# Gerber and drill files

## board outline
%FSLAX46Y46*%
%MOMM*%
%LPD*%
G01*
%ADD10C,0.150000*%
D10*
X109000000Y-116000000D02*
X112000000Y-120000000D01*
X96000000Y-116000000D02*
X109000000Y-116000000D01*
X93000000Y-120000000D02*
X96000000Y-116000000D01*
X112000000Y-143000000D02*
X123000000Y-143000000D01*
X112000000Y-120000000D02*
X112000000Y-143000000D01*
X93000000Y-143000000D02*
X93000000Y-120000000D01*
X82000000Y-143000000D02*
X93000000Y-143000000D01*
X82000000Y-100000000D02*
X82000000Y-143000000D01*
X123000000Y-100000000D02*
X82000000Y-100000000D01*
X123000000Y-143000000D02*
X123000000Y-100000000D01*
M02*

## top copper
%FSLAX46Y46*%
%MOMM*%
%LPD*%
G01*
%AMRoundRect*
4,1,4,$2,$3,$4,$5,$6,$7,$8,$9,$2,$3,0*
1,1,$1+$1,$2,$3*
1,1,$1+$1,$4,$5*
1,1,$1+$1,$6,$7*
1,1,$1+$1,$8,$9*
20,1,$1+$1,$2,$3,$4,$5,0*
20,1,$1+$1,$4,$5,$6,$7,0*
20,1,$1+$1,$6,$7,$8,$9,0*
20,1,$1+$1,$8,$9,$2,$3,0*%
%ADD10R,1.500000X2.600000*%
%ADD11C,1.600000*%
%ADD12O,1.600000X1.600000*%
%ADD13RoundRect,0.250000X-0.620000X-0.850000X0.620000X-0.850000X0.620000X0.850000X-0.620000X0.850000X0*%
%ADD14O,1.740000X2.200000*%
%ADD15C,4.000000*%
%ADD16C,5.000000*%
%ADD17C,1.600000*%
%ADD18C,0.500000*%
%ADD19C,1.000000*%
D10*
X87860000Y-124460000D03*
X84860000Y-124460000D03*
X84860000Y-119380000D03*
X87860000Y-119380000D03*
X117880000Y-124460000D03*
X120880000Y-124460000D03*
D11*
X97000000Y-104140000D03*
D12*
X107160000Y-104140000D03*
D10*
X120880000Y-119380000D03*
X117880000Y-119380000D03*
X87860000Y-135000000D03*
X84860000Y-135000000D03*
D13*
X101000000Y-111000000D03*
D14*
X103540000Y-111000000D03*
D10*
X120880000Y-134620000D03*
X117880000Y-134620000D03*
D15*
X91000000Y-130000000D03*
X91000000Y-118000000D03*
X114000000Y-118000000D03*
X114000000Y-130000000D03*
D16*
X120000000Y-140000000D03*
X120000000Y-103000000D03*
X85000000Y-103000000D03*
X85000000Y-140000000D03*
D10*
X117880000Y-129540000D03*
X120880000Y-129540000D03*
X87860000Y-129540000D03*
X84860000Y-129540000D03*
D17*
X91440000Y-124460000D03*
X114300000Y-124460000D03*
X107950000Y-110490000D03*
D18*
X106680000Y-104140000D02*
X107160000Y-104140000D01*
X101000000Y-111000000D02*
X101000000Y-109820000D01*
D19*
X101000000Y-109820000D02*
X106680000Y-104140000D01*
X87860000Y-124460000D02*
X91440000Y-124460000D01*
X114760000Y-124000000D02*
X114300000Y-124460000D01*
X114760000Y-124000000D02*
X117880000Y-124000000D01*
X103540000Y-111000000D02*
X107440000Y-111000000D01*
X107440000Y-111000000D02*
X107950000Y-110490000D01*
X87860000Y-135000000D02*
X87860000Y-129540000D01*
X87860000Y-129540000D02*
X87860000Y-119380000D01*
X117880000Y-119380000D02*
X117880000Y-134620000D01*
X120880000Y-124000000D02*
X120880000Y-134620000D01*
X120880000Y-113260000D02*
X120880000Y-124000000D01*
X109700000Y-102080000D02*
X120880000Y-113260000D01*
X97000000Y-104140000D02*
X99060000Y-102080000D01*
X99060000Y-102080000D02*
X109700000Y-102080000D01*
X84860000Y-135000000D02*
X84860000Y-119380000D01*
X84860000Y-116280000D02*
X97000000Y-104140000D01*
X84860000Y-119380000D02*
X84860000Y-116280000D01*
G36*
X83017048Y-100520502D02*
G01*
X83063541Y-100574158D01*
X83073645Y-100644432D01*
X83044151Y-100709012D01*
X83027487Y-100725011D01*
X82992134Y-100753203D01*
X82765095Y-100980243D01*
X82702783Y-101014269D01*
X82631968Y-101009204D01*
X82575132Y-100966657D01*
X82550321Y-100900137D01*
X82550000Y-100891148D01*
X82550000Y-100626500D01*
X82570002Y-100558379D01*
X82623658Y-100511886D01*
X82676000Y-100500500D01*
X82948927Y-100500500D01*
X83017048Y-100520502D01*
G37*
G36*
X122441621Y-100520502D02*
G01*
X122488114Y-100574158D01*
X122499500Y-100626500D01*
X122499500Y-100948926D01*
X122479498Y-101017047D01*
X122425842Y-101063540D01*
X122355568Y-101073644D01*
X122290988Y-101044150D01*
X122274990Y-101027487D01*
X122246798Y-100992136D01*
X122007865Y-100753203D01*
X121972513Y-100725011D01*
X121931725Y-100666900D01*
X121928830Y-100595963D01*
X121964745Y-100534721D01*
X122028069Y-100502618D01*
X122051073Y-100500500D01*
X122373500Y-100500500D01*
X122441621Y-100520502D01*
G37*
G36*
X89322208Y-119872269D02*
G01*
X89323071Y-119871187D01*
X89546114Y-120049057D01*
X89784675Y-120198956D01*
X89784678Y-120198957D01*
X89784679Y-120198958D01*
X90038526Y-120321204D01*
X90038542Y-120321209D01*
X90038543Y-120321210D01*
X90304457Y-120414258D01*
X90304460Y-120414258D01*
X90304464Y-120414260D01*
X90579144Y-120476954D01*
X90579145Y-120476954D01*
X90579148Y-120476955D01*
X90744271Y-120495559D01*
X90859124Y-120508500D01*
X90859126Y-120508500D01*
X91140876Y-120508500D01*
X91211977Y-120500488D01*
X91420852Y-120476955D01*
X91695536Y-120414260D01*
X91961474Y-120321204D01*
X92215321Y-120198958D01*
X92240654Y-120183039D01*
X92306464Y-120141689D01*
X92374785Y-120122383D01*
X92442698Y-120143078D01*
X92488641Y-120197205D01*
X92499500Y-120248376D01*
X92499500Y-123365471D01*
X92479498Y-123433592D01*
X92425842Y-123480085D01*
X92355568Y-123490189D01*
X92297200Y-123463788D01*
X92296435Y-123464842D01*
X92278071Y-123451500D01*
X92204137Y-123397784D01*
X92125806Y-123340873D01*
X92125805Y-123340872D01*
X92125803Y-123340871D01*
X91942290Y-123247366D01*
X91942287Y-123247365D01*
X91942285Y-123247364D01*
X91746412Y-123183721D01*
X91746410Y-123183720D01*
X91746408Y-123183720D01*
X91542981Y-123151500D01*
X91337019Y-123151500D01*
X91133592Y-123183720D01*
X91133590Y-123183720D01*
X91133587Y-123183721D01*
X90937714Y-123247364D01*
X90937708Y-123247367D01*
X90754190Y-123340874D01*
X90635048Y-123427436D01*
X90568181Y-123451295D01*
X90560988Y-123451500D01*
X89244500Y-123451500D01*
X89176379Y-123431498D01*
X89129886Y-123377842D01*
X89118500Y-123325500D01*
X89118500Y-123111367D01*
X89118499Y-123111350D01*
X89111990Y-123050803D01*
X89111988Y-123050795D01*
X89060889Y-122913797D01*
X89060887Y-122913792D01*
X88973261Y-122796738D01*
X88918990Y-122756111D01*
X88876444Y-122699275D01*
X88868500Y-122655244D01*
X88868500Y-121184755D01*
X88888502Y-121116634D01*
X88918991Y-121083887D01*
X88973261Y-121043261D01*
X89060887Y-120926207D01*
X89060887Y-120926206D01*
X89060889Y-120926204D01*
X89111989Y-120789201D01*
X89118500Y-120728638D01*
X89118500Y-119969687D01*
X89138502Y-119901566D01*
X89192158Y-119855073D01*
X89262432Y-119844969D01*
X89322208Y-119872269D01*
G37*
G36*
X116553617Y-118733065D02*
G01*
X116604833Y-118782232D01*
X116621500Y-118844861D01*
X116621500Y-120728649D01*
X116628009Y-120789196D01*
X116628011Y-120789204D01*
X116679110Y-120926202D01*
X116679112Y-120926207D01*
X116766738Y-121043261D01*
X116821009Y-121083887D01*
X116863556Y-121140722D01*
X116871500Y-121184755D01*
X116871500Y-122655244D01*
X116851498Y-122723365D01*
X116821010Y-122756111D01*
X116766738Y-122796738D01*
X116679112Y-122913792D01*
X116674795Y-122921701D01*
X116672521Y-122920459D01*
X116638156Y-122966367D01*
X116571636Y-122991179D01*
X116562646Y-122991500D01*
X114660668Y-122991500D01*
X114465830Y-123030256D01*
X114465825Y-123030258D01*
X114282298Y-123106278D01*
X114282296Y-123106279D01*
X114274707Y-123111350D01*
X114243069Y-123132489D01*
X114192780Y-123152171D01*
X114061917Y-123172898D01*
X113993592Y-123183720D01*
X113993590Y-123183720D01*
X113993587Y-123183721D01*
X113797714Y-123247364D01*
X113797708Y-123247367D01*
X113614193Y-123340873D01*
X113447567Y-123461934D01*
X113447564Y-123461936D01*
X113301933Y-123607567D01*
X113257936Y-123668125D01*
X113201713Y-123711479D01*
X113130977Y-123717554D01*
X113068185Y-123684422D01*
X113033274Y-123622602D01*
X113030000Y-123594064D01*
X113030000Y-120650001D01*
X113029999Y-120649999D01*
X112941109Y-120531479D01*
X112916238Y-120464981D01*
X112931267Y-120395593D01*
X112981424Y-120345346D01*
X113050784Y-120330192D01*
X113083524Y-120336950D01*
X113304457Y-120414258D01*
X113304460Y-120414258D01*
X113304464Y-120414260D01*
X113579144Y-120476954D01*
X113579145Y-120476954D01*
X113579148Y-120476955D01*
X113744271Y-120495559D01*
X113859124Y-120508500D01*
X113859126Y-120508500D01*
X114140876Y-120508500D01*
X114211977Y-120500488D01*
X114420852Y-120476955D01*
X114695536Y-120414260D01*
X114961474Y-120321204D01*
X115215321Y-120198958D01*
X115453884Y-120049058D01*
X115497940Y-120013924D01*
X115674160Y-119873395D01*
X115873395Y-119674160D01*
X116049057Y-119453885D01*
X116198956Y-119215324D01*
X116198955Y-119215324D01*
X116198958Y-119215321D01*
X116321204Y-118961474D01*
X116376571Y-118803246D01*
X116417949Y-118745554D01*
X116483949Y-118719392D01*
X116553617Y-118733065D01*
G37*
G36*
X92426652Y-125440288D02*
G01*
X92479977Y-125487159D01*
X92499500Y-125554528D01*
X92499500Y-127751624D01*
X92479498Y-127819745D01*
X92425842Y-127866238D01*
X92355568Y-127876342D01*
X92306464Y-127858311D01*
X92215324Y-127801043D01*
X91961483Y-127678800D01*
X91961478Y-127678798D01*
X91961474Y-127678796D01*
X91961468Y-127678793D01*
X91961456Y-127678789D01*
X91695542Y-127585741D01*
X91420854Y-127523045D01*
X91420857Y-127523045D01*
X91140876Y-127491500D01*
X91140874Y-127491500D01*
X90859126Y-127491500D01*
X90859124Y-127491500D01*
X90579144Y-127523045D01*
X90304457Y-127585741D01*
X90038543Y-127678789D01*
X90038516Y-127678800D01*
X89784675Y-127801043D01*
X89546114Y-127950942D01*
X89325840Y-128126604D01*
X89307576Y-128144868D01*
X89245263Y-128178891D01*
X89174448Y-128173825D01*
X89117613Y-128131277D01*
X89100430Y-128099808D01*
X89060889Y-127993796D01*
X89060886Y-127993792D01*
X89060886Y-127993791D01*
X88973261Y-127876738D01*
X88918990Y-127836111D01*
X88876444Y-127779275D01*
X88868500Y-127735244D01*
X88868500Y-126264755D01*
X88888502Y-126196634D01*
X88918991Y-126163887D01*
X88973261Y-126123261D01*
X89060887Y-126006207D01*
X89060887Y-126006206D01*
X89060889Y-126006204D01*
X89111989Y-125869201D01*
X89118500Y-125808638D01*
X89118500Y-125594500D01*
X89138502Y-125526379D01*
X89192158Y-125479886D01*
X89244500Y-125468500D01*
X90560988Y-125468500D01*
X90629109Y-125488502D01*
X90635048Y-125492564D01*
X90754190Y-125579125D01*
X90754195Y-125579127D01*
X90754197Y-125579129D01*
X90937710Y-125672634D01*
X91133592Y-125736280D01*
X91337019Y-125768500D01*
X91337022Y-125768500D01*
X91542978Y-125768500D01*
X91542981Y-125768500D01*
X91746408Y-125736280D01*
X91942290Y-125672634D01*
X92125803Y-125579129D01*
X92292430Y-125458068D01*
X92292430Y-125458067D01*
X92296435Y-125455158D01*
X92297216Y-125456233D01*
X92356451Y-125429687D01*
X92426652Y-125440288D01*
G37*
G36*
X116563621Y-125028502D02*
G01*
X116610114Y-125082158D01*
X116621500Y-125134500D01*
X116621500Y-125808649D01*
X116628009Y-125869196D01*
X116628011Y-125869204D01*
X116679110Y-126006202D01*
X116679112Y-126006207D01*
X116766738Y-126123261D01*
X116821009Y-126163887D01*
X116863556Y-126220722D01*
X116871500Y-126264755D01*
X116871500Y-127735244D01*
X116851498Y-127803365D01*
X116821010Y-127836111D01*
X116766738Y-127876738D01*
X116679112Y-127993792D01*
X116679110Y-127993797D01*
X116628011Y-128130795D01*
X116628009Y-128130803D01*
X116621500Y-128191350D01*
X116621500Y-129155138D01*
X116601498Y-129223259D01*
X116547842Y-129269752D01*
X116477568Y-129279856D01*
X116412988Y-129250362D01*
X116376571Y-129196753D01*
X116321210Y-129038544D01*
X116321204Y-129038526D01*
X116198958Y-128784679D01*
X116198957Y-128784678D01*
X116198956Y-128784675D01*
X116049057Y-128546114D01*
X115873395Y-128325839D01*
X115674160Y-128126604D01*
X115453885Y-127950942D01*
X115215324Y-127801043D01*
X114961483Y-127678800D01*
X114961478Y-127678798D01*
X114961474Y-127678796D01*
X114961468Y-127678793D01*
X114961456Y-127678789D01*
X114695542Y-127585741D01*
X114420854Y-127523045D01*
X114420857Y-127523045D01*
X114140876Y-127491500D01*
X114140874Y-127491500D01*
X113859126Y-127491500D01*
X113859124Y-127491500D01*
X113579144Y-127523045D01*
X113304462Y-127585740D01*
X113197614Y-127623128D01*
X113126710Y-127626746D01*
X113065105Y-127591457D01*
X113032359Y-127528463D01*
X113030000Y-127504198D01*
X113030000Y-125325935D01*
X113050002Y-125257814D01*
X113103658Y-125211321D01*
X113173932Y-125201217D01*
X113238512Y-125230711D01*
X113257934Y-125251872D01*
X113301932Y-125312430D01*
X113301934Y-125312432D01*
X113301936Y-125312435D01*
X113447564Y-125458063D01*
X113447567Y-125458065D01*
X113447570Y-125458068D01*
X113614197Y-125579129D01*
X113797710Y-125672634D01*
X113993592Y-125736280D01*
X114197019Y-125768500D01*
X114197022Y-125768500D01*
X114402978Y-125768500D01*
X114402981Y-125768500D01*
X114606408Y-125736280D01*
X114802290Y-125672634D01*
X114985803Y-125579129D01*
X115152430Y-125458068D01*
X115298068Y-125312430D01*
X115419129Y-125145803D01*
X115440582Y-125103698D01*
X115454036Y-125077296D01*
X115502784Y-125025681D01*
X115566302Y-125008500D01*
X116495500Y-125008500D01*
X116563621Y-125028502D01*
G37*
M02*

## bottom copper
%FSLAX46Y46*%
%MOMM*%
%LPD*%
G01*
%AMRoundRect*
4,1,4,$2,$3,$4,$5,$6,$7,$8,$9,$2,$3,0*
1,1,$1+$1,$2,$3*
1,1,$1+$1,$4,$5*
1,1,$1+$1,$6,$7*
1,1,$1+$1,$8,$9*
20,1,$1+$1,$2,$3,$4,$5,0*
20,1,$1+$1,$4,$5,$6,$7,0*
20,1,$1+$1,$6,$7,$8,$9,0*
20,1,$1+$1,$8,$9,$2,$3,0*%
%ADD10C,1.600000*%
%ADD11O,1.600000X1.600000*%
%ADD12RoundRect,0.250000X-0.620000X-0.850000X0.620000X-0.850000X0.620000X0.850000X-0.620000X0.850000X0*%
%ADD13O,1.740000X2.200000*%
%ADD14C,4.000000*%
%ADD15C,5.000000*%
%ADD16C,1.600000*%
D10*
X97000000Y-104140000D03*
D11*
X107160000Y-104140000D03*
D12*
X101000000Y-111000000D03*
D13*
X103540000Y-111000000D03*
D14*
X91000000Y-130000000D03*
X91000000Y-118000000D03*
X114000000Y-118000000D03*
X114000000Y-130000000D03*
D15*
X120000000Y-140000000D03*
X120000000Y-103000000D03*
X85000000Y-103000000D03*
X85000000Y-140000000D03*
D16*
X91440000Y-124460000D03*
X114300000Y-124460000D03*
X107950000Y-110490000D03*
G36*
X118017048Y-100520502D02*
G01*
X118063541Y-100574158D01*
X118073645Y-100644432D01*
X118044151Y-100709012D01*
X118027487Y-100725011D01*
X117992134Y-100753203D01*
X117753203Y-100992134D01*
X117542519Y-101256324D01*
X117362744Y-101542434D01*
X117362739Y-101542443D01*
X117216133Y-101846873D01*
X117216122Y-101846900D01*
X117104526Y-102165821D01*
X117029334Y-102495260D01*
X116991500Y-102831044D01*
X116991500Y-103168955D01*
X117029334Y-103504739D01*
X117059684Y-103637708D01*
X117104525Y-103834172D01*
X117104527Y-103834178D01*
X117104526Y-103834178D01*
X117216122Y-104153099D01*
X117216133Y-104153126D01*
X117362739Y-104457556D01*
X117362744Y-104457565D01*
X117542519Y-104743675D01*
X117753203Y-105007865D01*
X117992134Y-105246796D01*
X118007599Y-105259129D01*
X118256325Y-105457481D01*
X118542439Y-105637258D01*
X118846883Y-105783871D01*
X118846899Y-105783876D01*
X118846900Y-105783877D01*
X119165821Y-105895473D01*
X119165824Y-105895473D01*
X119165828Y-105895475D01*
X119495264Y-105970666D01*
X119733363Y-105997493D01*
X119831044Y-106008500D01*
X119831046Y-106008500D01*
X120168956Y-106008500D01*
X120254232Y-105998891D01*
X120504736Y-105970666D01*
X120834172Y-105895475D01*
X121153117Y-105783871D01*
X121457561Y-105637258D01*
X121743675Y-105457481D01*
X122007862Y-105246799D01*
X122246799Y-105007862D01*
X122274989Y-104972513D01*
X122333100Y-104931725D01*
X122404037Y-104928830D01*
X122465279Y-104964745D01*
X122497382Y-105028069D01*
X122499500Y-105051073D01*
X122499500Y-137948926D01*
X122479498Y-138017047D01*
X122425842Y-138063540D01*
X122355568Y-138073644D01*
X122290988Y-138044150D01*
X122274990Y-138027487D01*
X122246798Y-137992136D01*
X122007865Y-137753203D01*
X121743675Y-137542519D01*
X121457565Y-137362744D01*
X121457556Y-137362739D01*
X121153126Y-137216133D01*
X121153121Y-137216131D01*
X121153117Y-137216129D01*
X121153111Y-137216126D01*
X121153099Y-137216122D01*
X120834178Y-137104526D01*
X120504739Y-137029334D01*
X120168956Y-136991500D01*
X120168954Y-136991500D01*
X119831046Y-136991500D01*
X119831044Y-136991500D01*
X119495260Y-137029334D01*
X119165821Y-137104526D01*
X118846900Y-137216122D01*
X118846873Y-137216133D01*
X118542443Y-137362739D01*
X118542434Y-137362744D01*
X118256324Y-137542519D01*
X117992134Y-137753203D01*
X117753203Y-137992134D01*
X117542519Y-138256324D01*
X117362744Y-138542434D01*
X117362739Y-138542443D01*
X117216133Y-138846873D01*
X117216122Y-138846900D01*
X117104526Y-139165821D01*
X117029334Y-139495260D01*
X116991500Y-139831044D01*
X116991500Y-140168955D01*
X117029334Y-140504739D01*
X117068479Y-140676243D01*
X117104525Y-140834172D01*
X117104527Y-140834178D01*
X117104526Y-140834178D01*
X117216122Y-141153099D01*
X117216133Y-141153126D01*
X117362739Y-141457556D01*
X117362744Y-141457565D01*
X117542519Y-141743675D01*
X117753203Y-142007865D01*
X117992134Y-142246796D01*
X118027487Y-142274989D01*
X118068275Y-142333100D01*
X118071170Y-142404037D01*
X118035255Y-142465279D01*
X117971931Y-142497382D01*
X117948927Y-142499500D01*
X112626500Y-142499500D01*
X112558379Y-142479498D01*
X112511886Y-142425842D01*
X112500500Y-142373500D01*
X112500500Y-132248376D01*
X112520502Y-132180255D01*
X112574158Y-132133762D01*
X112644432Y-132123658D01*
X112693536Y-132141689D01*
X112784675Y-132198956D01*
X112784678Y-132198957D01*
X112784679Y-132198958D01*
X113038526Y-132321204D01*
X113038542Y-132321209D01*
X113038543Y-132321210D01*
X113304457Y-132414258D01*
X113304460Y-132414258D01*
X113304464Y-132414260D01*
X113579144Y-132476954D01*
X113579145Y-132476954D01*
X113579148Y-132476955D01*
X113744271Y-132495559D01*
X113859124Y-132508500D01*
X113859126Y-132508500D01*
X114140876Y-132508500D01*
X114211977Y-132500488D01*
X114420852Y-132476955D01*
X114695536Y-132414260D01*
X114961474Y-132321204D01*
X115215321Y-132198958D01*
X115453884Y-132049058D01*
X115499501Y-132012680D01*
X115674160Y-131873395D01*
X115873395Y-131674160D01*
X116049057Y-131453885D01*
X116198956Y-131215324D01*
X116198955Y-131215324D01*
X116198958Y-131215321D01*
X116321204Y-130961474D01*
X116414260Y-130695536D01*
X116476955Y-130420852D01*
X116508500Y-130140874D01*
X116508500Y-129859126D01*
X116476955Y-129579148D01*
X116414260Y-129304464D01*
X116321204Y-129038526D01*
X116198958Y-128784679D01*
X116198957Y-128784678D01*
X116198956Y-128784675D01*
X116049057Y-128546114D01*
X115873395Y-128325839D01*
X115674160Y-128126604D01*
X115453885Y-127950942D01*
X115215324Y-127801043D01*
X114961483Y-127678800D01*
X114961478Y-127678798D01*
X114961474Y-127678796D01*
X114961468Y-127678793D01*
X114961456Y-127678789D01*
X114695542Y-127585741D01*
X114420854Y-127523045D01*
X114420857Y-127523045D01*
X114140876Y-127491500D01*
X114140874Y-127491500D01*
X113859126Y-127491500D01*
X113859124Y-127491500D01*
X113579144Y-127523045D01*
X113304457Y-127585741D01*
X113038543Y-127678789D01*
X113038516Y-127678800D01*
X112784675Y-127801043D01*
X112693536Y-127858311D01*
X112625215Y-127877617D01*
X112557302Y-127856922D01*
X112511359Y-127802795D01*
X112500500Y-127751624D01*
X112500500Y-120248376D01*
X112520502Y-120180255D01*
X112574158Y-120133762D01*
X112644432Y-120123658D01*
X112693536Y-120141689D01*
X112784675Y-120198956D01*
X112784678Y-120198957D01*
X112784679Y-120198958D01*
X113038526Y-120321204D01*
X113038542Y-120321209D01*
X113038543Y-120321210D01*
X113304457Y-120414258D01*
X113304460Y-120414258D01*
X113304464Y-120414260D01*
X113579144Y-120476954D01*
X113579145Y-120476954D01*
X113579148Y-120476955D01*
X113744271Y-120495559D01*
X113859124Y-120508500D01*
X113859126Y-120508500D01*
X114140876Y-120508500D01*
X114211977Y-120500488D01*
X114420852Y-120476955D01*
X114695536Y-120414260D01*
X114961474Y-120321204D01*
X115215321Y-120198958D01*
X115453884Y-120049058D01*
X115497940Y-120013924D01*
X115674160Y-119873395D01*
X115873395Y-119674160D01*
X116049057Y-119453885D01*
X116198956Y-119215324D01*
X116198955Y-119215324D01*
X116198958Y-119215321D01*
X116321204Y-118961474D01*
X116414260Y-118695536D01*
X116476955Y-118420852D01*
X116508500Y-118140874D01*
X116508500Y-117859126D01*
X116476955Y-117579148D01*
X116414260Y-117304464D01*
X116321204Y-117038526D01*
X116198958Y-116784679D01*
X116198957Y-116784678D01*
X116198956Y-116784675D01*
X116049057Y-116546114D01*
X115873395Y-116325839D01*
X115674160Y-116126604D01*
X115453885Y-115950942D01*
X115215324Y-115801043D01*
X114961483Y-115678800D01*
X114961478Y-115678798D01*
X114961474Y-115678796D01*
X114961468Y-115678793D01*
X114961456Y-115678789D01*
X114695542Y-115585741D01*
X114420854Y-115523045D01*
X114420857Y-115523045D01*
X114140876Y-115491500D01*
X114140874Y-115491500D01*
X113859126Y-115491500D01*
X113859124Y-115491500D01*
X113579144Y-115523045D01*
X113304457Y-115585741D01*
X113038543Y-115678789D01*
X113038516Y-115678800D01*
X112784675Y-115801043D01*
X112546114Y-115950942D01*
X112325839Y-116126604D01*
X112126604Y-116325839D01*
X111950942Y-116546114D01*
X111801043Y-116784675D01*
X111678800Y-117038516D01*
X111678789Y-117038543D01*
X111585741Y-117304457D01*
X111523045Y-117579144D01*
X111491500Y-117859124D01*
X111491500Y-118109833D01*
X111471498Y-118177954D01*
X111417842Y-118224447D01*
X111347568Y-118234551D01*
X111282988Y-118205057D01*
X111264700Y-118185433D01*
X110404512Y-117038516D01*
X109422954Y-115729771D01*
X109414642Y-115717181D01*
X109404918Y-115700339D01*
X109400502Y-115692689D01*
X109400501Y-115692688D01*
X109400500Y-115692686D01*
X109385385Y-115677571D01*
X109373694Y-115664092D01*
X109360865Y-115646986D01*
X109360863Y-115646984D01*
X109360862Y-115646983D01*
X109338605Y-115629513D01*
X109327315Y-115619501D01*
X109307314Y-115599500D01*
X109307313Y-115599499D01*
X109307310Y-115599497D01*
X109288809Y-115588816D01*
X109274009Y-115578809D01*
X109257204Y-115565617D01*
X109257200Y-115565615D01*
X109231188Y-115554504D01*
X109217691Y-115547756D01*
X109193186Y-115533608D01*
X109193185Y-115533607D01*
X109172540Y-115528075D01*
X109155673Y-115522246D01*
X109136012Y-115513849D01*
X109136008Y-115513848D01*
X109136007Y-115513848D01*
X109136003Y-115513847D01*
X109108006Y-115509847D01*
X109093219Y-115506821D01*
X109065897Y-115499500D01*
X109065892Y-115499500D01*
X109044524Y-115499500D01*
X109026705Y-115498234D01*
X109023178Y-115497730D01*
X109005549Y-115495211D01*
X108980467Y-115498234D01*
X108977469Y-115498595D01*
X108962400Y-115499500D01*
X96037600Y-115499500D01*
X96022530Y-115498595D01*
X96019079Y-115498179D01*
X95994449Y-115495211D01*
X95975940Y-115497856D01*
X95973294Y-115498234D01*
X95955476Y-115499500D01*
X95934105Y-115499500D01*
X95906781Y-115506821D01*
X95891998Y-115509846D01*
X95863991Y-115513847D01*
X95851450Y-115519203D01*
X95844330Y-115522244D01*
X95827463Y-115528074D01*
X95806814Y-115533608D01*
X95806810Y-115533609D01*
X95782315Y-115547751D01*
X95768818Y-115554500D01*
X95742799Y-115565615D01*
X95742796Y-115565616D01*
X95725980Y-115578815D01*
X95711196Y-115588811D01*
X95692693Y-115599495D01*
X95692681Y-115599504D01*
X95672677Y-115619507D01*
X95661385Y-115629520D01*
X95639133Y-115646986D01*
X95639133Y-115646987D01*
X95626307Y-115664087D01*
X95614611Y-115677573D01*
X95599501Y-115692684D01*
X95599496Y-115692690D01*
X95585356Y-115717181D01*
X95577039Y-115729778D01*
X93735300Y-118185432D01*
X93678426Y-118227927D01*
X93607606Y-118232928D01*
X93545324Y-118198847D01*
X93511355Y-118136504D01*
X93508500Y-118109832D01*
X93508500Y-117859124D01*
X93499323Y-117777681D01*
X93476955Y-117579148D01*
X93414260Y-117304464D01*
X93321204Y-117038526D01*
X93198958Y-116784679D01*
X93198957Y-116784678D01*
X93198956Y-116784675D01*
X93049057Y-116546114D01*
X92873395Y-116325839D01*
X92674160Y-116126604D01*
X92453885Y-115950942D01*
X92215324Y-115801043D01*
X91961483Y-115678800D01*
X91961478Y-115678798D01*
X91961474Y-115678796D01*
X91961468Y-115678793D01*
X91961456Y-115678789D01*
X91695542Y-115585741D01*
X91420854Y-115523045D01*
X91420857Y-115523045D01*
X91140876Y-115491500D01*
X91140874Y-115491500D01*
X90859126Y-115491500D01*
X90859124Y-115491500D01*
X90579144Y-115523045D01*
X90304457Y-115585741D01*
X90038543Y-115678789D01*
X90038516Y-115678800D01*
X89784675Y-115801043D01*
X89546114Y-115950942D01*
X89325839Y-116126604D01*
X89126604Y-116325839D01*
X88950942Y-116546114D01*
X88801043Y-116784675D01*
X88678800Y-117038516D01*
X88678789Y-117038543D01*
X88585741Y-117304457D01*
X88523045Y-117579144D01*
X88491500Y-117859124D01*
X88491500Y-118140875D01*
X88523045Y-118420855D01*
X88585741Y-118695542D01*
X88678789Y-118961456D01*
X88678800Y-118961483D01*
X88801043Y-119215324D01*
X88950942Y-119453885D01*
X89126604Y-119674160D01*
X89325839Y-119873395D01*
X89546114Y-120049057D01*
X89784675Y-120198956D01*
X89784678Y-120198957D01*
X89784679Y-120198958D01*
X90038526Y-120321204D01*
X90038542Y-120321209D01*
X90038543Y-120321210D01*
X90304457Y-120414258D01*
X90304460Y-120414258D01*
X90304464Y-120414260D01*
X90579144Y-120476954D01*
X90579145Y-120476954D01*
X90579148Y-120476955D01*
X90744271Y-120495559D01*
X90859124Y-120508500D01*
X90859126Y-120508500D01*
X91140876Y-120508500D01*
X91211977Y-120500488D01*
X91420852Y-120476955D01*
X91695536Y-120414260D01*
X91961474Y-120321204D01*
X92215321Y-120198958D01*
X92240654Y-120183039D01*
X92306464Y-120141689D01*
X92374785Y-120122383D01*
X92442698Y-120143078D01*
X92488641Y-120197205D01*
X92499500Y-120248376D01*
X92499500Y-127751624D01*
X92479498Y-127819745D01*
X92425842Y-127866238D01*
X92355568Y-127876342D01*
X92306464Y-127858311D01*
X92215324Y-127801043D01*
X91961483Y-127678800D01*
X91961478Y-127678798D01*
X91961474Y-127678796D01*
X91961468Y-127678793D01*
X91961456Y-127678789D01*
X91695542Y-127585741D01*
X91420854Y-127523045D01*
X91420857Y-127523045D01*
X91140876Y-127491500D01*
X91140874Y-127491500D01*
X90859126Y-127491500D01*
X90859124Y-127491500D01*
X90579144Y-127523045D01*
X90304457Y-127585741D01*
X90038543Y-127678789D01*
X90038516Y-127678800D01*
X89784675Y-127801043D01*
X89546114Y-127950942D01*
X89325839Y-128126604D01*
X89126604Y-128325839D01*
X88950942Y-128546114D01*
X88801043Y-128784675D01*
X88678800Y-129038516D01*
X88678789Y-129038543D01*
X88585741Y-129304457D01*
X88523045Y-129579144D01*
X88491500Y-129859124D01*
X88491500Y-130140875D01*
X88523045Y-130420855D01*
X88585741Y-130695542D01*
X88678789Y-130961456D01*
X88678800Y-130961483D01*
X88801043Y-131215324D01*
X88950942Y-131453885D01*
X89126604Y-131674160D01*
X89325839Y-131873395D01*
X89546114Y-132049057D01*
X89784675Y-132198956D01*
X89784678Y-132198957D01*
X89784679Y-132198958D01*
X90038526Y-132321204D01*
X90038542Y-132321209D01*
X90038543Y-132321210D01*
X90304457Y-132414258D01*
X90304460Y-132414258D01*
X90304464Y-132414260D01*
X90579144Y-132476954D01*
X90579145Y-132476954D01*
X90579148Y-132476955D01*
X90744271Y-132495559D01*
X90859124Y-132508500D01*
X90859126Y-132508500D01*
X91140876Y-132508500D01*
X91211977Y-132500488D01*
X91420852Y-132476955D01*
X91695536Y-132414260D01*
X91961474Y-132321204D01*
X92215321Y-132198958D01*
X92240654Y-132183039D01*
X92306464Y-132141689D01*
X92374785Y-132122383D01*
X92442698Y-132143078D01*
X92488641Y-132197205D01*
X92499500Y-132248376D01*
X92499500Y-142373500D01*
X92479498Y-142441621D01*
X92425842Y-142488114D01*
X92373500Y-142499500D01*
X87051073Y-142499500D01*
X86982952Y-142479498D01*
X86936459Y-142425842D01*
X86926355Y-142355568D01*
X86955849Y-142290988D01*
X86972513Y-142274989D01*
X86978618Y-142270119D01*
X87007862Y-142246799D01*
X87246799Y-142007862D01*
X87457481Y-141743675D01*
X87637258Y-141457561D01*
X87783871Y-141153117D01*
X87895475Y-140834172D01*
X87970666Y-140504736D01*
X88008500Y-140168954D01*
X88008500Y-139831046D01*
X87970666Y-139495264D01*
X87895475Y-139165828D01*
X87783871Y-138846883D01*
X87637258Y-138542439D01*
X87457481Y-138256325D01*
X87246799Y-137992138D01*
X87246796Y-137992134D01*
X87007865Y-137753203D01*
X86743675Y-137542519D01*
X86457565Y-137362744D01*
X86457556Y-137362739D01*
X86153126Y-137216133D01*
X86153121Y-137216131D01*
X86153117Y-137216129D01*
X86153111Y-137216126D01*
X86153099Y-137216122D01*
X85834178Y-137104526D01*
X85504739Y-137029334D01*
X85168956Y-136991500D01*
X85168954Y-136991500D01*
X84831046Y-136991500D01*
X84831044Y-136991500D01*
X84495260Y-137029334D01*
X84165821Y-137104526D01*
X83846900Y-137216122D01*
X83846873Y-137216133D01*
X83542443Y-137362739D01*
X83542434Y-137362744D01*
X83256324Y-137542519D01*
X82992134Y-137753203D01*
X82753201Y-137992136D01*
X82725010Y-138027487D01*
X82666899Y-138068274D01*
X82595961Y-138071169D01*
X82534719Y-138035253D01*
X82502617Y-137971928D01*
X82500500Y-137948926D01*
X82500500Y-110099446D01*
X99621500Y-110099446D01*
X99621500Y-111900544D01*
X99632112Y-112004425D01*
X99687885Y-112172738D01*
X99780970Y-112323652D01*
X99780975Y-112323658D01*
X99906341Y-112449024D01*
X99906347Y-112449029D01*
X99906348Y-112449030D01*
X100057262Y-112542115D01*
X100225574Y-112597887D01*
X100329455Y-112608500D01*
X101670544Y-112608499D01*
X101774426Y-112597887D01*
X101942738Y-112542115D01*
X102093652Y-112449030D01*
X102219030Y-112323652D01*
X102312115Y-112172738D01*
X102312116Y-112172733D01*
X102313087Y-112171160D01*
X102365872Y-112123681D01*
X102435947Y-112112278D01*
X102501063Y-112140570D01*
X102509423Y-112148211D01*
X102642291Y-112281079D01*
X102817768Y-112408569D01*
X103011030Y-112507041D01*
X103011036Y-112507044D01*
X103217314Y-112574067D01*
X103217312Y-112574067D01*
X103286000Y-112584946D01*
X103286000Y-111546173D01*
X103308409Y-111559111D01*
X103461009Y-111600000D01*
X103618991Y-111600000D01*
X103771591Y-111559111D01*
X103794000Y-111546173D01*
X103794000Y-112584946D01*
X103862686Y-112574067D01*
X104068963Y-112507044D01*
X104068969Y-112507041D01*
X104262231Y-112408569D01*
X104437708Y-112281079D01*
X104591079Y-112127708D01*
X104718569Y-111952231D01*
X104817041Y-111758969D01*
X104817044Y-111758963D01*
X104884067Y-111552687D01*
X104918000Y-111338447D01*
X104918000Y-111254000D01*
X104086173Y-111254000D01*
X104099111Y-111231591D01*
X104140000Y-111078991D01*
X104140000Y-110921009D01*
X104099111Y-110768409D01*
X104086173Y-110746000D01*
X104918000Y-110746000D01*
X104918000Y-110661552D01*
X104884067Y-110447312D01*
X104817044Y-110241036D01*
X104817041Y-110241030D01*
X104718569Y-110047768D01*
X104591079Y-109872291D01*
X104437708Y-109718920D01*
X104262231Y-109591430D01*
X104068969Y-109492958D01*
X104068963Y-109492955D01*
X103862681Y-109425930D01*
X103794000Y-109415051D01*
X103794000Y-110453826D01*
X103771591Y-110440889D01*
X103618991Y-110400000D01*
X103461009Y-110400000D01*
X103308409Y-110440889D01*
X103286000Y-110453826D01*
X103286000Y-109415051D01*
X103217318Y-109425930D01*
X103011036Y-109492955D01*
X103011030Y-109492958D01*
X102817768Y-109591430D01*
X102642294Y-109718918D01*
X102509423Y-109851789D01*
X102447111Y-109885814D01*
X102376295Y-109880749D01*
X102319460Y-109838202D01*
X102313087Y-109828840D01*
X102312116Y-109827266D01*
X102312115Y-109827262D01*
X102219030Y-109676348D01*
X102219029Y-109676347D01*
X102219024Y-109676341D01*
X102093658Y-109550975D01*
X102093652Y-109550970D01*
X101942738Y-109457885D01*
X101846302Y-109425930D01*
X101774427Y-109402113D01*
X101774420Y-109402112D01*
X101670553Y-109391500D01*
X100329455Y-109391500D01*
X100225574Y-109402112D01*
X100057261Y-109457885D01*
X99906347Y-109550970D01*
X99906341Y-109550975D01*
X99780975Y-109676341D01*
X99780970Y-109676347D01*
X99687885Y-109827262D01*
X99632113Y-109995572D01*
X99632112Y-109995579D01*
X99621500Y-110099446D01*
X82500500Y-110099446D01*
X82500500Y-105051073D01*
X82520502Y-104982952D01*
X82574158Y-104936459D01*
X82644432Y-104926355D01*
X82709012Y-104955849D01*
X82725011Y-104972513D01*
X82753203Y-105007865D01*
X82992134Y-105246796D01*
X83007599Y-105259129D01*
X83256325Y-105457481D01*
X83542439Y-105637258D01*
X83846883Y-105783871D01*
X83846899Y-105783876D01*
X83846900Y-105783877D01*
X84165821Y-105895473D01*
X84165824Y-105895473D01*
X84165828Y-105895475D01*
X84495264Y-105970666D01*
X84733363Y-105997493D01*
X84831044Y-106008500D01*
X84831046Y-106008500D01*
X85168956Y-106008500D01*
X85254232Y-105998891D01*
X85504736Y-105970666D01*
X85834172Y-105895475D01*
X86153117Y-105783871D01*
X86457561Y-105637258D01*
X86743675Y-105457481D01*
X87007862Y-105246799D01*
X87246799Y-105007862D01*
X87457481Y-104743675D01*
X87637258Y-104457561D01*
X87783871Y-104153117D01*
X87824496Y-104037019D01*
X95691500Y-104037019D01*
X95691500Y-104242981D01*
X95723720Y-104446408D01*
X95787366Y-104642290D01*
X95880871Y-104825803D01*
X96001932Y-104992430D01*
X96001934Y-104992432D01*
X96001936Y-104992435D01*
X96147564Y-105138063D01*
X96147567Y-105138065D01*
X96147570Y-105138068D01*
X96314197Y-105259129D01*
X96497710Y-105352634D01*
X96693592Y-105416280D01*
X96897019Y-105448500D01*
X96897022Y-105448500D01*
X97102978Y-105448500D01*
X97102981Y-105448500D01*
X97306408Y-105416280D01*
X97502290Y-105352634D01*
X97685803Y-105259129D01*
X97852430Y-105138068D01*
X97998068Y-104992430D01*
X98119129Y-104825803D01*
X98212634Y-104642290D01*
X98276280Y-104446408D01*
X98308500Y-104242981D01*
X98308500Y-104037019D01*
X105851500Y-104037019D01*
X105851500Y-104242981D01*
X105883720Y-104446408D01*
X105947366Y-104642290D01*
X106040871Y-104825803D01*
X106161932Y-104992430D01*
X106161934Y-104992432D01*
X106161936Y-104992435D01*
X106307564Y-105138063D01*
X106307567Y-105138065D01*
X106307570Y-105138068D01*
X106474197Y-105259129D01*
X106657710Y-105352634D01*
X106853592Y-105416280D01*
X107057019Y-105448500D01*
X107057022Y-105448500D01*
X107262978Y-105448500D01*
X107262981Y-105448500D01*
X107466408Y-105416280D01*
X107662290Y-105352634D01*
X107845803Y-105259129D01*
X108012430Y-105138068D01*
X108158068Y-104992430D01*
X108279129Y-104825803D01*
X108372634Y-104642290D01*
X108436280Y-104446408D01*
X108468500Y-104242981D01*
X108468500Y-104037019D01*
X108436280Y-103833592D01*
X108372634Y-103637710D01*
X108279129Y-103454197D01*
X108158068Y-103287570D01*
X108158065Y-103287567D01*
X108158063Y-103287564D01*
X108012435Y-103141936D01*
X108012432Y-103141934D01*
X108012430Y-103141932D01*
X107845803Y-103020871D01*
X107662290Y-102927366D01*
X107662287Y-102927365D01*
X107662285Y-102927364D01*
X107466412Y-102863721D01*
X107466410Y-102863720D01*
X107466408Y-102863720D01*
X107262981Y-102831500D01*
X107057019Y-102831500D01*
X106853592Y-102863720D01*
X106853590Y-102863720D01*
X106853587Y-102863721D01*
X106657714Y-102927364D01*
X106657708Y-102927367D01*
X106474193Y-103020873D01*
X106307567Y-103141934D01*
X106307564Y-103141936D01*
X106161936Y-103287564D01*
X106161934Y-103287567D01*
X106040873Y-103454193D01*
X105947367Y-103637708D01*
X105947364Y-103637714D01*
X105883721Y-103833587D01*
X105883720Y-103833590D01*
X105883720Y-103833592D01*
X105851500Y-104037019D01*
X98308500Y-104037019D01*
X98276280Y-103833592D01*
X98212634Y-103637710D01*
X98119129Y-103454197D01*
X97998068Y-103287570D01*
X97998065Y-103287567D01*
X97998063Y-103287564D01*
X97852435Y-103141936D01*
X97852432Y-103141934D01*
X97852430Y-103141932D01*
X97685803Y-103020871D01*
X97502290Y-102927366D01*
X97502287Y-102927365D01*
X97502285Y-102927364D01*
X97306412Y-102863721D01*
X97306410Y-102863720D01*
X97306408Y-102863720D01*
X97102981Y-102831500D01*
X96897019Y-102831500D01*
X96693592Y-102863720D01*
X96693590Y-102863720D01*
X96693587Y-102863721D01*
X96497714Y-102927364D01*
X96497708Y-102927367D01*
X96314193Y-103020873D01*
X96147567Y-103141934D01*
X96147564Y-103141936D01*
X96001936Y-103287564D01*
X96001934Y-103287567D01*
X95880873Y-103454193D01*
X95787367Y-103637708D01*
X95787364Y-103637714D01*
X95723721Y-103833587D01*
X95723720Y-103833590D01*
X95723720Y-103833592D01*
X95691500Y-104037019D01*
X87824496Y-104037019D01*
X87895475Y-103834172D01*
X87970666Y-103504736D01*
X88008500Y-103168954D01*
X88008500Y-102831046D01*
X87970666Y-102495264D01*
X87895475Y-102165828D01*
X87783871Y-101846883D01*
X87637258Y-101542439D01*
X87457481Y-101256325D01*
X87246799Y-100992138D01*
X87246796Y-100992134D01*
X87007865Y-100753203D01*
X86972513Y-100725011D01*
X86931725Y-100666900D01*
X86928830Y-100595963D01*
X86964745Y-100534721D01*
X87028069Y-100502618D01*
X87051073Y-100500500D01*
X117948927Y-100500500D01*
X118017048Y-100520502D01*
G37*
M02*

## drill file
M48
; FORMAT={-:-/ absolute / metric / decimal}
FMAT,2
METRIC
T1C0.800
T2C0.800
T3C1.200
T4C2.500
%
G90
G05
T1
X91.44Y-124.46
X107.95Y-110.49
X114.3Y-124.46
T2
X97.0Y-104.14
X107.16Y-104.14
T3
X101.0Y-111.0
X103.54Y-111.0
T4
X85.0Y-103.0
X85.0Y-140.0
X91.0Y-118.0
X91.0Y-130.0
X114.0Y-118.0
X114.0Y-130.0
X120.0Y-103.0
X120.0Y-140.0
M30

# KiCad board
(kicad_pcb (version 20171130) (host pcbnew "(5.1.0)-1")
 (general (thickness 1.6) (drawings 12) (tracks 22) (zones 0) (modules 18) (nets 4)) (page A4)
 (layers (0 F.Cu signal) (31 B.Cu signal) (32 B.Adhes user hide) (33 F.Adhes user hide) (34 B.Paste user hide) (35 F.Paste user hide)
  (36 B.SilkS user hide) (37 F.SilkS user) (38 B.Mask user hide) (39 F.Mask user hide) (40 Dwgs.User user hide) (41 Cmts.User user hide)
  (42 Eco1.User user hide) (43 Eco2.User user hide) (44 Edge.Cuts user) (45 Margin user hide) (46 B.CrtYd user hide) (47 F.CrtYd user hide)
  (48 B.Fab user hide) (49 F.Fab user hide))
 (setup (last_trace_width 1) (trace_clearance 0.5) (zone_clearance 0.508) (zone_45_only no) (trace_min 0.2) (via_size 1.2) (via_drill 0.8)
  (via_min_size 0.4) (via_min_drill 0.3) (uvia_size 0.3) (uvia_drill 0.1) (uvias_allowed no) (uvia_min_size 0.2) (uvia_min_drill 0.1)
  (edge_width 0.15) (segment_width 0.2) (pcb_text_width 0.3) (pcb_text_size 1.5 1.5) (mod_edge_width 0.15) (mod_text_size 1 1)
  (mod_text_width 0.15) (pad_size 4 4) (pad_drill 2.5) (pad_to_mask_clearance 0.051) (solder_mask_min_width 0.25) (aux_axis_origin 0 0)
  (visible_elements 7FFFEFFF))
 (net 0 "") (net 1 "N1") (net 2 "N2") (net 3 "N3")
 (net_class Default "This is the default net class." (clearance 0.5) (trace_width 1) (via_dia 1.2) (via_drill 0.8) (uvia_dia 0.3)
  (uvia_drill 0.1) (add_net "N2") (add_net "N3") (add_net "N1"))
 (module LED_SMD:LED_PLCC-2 (layer F.Cu) (at 86.36 124.46 180)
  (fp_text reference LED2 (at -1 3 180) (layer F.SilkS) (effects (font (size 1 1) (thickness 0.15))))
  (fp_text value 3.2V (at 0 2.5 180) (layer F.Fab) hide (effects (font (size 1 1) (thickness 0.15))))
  (pad 1 smd rect (at -1.5 0 180) (size 1.5 2.6) (layers F.Cu F.Paste F.Mask) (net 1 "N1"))
  (pad 2 smd rect (at 1.5 0 180) (size 1.5 2.6) (layers F.Cu F.Paste F.Mask) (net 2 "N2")))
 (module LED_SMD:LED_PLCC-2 (layer F.Cu) (at 86.36 119.38 180)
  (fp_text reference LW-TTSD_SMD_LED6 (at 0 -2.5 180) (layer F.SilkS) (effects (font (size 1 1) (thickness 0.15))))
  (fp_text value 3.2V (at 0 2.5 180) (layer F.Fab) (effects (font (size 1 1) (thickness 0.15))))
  (pad 2 smd rect (at 1.5 0 180) (size 1.5 2.6) (layers F.Cu F.Paste F.Mask) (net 2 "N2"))
  (pad 1 smd rect (at -1.5 0 180) (size 1.5 2.6) (layers F.Cu F.Paste F.Mask) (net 1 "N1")))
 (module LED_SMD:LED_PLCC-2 (layer F.Cu) (at 119.38 124.46)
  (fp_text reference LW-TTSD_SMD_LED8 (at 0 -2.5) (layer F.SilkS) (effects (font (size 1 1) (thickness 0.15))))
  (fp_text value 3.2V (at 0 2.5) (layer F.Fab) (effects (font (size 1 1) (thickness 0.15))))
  (pad 1 smd rect (at -1.5 0) (size 1.5 2.6) (layers F.Cu F.Paste F.Mask) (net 1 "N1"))
  (pad 2 smd rect (at 1.5 0) (size 1.5 2.6) (layers F.Cu F.Paste F.Mask) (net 2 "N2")))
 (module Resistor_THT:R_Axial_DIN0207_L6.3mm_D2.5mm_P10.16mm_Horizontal (layer F.Cu) (at 97 104.14)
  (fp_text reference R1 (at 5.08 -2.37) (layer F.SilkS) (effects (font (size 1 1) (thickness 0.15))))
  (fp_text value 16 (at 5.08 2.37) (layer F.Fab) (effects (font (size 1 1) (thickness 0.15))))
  (pad 1 thru_hole circle (at 0 0) (size 1.6 1.6) (drill 0.8) (layers *.Cu *.Mask) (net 2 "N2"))
  (pad 2 thru_hole oval (at 10.16 0) (size 1.6 1.6) (drill 0.8) (layers *.Cu *.Mask) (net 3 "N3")))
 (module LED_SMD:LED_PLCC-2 (layer F.Cu) (at 119.38 119.38)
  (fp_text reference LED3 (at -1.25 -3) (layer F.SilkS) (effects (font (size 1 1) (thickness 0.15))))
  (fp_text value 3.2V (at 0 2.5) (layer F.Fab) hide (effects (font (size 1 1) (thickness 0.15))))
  (pad 2 smd rect (at 1.5 0) (size 1.5 2.6) (layers F.Cu F.Paste F.Mask) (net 2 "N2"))
  (pad 1 smd rect (at -1.5 0) (size 1.5 2.6) (layers F.Cu F.Paste F.Mask) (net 1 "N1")))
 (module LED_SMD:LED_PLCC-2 (layer F.Cu) (at 86.36 135 180)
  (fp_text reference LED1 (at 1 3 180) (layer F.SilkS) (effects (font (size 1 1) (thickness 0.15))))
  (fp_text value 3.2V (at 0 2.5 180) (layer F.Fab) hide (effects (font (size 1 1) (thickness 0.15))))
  (pad 1 smd rect (at -1.5 0 180) (size 1.5 2.6) (layers F.Cu F.Paste F.Mask) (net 1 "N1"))
  (pad 2 smd rect (at 1.5 0 180) (size 1.5 2.6) (layers F.Cu F.Paste F.Mask) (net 2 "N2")))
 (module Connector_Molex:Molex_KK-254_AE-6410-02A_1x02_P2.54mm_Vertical (layer B.Cu) (at 101 111)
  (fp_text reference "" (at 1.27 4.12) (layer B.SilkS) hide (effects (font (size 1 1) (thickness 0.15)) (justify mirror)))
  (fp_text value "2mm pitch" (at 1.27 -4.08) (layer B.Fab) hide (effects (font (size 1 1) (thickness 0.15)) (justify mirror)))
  (pad 1 thru_hole roundrect (at 0 0) (size 1.74 2.2) (drill 1.2) (layers *.Cu *.Mask) (roundrect_rratio 0.143678) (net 3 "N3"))
  (pad 2 thru_hole oval (at 2.54 0) (size 1.74 2.2) (drill 1.2) (layers *.Cu *.Mask) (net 1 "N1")))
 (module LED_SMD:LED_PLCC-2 (layer F.Cu) (at 119.38 134.62)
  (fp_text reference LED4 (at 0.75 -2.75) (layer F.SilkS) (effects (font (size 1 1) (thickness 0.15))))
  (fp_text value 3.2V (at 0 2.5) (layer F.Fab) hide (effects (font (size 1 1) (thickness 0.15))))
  (pad 2 smd rect (at 1.5 0) (size 1.5 2.6) (layers F.Cu F.Paste F.Mask) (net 2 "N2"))
  (pad 1 smd rect (at -1.5 0) (size 1.5 2.6) (layers F.Cu F.Paste F.Mask) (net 1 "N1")))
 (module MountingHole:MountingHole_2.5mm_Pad (layer F.Cu) (at 91 130)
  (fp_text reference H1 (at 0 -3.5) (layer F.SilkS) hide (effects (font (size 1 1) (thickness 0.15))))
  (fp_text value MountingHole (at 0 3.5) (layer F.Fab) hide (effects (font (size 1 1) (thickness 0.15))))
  (pad 1 thru_hole circle (at 0 0) (size 4 4) (drill 2.5) (layers *.Cu *.Mask)))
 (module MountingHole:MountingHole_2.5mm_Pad (layer F.Cu) (at 91 118)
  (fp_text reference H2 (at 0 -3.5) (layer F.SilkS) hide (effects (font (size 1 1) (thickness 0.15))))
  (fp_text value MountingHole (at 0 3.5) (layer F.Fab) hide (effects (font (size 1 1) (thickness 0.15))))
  (pad 1 thru_hole circle (at 0 0) (size 4 4) (drill 2.5) (layers *.Cu *.Mask)))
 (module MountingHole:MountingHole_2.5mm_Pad (layer F.Cu) (at 114 118)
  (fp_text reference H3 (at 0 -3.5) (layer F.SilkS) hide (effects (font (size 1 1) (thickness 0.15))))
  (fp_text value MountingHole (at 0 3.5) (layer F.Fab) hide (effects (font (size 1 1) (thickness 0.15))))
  (pad 1 thru_hole circle (at 0 0) (size 4 4) (drill 2.5) (layers *.Cu *.Mask)))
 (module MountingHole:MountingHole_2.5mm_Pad (layer F.Cu) (at 114 130)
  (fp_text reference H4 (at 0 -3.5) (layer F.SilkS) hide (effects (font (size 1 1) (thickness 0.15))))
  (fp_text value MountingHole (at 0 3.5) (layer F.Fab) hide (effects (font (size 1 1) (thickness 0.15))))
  (pad 1 thru_hole circle (at 0 0) (size 4 4) (drill 2.5) (layers *.Cu *.Mask)))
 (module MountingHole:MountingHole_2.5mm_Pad (layer F.Cu) (at 120 140)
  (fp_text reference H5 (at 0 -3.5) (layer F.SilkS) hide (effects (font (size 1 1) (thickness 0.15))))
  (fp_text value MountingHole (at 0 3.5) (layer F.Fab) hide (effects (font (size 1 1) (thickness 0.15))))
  (pad 1 thru_hole circle (at 0 0) (size 5 5) (drill 2.5) (layers *.Cu *.Mask)))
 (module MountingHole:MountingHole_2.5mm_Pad (layer F.Cu) (at 120 103)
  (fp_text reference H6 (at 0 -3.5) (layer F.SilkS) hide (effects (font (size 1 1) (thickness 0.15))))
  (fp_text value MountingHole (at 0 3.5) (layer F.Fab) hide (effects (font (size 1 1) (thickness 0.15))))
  (pad 1 thru_hole circle (at 0 0) (size 5 5) (drill 2.5) (layers *.Cu *.Mask)))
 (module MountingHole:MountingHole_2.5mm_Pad (layer F.Cu) (at 85 103)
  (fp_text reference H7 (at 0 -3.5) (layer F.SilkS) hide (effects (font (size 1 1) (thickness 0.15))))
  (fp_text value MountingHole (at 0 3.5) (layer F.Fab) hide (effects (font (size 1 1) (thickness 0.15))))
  (pad 1 thru_hole circle (at 0 0) (size 5 5) (drill 2.5) (layers *.Cu *.Mask)))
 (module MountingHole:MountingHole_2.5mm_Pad (layer F.Cu) (at 85 140)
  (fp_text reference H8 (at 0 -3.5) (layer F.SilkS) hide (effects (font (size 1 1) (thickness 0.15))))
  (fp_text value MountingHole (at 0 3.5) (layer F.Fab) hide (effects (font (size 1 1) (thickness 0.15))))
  (pad 1 thru_hole circle (at 0 0) (size 5 5) (drill 2.5) (layers *.Cu *.Mask)))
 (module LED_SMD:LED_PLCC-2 (layer F.Cu) (at 119.38 129.54)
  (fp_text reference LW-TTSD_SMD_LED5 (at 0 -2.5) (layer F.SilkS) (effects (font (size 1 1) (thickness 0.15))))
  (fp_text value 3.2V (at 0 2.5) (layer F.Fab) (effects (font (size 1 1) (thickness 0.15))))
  (pad 1 smd rect (at -1.5 0) (size 1.5 2.6) (layers F.Cu F.Paste F.Mask) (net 1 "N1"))
  (pad 2 smd rect (at 1.5 0) (size 1.5 2.6) (layers F.Cu F.Paste F.Mask) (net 2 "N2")))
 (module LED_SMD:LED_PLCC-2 (layer F.Cu) (at 86.36 129.54 180)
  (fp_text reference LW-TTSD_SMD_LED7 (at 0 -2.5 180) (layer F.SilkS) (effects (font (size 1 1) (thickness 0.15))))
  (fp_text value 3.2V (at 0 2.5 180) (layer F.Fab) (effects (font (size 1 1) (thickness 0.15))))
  (pad 1 smd rect (at -1.5 0 180) (size 1.5 2.6) (layers F.Cu F.Paste F.Mask) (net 1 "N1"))
  (pad 2 smd rect (at 1.5 0 180) (size 1.5 2.6) (layers F.Cu F.Paste F.Mask) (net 2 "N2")))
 (gr_line (start 109 116) (end 112 120) (layer Edge.Cuts) (width 0.15))
 (gr_line (start 96 116) (end 109 116) (layer Edge.Cuts) (width 0.15))
 (gr_line (start 93 120) (end 96 116) (layer Edge.Cuts) (width 0.15))
 (gr_line (start 112 143) (end 123 143) (layer Edge.Cuts) (width 0.15))
 (gr_line (start 112 120) (end 112 143) (layer Edge.Cuts) (width 0.15))
 (gr_line (start 93 143) (end 93 120) (layer Edge.Cuts) (width 0.15))
 (gr_line (start 82 143) (end 93 143) (layer Edge.Cuts) (width 0.15))
 (gr_line (start 82 100) (end 82 143) (layer Edge.Cuts) (width 0.15))
 (gr_line (start 123 100) (end 82 100) (layer Edge.Cuts) (width 0.15))
 (gr_line (start 123 143) (end 123 100) (layer Edge.Cuts) (width 0.15))
 (segment (start 106.68 104.14) (end 107.16 104.14) (width 0.5) (layer F.Cu) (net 3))
 (segment (start 101 111) (end 101 109.82) (width 0.5) (layer F.Cu) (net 3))
 (segment (start 101 109.82) (end 106.68 104.14) (width 1) (layer F.Cu) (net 3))
 (via (at 91.44 124.46) (size 1.6) (drill 0.8) (layers F.Cu B.Cu) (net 1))
 (segment (start 87.86 124.46) (end 91.44 124.46) (width 1) (layer F.Cu) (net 1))
 (via (at 114.3 124.46) (size 1.6) (drill 0.8) (layers F.Cu B.Cu) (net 1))
 (segment (start 114.76 124) (end 114.3 124.46) (width 1) (layer F.Cu) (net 1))
 (segment (start 114.76 124) (end 117.88 124) (width 1) (layer F.Cu) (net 1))
 (via (at 107.95 110.49) (size 1.6) (drill 0.8) (layers F.Cu B.Cu) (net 1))
 (segment (start 103.54 111) (end 107.44 111) (width 1) (layer F.Cu) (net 1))
 (segment (start 107.44 111) (end 107.95 110.49) (width 1) (layer F.Cu) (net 1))
 (segment (start 87.86 135) (end 87.86 129.54) (width 1) (layer F.Cu) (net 1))
 (segment (start 87.86 129.54) (end 87.86 119.38) (width 1) (layer F.Cu) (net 1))
 (segment (start 117.88 119.38) (end 117.88 134.62) (width 1) (layer F.Cu) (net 1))
 (segment (start 120.88 124) (end 120.88 134.62) (width 1) (layer F.Cu) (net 2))
 (segment (start 120.88 113.26) (end 120.88 124) (width 1) (layer F.Cu) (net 2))
 (segment (start 109.7 102.08) (end 120.88 113.26) (width 1) (layer F.Cu) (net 2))
 (segment (start 97 104.14) (end 99.06 102.08) (width 1) (layer F.Cu) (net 2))
 (segment (start 99.06 102.08) (end 109.7 102.08) (width 1) (layer F.Cu) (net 2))
 (segment (start 84.86 135) (end 84.86 119.38) (width 1) (layer F.Cu) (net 2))
 (segment (start 84.86 116.28) (end 97 104.14) (width 1) (layer F.Cu) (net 2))
 (segment (start 84.86 119.38) (end 84.86 116.28) (width 1) (layer F.Cu) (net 2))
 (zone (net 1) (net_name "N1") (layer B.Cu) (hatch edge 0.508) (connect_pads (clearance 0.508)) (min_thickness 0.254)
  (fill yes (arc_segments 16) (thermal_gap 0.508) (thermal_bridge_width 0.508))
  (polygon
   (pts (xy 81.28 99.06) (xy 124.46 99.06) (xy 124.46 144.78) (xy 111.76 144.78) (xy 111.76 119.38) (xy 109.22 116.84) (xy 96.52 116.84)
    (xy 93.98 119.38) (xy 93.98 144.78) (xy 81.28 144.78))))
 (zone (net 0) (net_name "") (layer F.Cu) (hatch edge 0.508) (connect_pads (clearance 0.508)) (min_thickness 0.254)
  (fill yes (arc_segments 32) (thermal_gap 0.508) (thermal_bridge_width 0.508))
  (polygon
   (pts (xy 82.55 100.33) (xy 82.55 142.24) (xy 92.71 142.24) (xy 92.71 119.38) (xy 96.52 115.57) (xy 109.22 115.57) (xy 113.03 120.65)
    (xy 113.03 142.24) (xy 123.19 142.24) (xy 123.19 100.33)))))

